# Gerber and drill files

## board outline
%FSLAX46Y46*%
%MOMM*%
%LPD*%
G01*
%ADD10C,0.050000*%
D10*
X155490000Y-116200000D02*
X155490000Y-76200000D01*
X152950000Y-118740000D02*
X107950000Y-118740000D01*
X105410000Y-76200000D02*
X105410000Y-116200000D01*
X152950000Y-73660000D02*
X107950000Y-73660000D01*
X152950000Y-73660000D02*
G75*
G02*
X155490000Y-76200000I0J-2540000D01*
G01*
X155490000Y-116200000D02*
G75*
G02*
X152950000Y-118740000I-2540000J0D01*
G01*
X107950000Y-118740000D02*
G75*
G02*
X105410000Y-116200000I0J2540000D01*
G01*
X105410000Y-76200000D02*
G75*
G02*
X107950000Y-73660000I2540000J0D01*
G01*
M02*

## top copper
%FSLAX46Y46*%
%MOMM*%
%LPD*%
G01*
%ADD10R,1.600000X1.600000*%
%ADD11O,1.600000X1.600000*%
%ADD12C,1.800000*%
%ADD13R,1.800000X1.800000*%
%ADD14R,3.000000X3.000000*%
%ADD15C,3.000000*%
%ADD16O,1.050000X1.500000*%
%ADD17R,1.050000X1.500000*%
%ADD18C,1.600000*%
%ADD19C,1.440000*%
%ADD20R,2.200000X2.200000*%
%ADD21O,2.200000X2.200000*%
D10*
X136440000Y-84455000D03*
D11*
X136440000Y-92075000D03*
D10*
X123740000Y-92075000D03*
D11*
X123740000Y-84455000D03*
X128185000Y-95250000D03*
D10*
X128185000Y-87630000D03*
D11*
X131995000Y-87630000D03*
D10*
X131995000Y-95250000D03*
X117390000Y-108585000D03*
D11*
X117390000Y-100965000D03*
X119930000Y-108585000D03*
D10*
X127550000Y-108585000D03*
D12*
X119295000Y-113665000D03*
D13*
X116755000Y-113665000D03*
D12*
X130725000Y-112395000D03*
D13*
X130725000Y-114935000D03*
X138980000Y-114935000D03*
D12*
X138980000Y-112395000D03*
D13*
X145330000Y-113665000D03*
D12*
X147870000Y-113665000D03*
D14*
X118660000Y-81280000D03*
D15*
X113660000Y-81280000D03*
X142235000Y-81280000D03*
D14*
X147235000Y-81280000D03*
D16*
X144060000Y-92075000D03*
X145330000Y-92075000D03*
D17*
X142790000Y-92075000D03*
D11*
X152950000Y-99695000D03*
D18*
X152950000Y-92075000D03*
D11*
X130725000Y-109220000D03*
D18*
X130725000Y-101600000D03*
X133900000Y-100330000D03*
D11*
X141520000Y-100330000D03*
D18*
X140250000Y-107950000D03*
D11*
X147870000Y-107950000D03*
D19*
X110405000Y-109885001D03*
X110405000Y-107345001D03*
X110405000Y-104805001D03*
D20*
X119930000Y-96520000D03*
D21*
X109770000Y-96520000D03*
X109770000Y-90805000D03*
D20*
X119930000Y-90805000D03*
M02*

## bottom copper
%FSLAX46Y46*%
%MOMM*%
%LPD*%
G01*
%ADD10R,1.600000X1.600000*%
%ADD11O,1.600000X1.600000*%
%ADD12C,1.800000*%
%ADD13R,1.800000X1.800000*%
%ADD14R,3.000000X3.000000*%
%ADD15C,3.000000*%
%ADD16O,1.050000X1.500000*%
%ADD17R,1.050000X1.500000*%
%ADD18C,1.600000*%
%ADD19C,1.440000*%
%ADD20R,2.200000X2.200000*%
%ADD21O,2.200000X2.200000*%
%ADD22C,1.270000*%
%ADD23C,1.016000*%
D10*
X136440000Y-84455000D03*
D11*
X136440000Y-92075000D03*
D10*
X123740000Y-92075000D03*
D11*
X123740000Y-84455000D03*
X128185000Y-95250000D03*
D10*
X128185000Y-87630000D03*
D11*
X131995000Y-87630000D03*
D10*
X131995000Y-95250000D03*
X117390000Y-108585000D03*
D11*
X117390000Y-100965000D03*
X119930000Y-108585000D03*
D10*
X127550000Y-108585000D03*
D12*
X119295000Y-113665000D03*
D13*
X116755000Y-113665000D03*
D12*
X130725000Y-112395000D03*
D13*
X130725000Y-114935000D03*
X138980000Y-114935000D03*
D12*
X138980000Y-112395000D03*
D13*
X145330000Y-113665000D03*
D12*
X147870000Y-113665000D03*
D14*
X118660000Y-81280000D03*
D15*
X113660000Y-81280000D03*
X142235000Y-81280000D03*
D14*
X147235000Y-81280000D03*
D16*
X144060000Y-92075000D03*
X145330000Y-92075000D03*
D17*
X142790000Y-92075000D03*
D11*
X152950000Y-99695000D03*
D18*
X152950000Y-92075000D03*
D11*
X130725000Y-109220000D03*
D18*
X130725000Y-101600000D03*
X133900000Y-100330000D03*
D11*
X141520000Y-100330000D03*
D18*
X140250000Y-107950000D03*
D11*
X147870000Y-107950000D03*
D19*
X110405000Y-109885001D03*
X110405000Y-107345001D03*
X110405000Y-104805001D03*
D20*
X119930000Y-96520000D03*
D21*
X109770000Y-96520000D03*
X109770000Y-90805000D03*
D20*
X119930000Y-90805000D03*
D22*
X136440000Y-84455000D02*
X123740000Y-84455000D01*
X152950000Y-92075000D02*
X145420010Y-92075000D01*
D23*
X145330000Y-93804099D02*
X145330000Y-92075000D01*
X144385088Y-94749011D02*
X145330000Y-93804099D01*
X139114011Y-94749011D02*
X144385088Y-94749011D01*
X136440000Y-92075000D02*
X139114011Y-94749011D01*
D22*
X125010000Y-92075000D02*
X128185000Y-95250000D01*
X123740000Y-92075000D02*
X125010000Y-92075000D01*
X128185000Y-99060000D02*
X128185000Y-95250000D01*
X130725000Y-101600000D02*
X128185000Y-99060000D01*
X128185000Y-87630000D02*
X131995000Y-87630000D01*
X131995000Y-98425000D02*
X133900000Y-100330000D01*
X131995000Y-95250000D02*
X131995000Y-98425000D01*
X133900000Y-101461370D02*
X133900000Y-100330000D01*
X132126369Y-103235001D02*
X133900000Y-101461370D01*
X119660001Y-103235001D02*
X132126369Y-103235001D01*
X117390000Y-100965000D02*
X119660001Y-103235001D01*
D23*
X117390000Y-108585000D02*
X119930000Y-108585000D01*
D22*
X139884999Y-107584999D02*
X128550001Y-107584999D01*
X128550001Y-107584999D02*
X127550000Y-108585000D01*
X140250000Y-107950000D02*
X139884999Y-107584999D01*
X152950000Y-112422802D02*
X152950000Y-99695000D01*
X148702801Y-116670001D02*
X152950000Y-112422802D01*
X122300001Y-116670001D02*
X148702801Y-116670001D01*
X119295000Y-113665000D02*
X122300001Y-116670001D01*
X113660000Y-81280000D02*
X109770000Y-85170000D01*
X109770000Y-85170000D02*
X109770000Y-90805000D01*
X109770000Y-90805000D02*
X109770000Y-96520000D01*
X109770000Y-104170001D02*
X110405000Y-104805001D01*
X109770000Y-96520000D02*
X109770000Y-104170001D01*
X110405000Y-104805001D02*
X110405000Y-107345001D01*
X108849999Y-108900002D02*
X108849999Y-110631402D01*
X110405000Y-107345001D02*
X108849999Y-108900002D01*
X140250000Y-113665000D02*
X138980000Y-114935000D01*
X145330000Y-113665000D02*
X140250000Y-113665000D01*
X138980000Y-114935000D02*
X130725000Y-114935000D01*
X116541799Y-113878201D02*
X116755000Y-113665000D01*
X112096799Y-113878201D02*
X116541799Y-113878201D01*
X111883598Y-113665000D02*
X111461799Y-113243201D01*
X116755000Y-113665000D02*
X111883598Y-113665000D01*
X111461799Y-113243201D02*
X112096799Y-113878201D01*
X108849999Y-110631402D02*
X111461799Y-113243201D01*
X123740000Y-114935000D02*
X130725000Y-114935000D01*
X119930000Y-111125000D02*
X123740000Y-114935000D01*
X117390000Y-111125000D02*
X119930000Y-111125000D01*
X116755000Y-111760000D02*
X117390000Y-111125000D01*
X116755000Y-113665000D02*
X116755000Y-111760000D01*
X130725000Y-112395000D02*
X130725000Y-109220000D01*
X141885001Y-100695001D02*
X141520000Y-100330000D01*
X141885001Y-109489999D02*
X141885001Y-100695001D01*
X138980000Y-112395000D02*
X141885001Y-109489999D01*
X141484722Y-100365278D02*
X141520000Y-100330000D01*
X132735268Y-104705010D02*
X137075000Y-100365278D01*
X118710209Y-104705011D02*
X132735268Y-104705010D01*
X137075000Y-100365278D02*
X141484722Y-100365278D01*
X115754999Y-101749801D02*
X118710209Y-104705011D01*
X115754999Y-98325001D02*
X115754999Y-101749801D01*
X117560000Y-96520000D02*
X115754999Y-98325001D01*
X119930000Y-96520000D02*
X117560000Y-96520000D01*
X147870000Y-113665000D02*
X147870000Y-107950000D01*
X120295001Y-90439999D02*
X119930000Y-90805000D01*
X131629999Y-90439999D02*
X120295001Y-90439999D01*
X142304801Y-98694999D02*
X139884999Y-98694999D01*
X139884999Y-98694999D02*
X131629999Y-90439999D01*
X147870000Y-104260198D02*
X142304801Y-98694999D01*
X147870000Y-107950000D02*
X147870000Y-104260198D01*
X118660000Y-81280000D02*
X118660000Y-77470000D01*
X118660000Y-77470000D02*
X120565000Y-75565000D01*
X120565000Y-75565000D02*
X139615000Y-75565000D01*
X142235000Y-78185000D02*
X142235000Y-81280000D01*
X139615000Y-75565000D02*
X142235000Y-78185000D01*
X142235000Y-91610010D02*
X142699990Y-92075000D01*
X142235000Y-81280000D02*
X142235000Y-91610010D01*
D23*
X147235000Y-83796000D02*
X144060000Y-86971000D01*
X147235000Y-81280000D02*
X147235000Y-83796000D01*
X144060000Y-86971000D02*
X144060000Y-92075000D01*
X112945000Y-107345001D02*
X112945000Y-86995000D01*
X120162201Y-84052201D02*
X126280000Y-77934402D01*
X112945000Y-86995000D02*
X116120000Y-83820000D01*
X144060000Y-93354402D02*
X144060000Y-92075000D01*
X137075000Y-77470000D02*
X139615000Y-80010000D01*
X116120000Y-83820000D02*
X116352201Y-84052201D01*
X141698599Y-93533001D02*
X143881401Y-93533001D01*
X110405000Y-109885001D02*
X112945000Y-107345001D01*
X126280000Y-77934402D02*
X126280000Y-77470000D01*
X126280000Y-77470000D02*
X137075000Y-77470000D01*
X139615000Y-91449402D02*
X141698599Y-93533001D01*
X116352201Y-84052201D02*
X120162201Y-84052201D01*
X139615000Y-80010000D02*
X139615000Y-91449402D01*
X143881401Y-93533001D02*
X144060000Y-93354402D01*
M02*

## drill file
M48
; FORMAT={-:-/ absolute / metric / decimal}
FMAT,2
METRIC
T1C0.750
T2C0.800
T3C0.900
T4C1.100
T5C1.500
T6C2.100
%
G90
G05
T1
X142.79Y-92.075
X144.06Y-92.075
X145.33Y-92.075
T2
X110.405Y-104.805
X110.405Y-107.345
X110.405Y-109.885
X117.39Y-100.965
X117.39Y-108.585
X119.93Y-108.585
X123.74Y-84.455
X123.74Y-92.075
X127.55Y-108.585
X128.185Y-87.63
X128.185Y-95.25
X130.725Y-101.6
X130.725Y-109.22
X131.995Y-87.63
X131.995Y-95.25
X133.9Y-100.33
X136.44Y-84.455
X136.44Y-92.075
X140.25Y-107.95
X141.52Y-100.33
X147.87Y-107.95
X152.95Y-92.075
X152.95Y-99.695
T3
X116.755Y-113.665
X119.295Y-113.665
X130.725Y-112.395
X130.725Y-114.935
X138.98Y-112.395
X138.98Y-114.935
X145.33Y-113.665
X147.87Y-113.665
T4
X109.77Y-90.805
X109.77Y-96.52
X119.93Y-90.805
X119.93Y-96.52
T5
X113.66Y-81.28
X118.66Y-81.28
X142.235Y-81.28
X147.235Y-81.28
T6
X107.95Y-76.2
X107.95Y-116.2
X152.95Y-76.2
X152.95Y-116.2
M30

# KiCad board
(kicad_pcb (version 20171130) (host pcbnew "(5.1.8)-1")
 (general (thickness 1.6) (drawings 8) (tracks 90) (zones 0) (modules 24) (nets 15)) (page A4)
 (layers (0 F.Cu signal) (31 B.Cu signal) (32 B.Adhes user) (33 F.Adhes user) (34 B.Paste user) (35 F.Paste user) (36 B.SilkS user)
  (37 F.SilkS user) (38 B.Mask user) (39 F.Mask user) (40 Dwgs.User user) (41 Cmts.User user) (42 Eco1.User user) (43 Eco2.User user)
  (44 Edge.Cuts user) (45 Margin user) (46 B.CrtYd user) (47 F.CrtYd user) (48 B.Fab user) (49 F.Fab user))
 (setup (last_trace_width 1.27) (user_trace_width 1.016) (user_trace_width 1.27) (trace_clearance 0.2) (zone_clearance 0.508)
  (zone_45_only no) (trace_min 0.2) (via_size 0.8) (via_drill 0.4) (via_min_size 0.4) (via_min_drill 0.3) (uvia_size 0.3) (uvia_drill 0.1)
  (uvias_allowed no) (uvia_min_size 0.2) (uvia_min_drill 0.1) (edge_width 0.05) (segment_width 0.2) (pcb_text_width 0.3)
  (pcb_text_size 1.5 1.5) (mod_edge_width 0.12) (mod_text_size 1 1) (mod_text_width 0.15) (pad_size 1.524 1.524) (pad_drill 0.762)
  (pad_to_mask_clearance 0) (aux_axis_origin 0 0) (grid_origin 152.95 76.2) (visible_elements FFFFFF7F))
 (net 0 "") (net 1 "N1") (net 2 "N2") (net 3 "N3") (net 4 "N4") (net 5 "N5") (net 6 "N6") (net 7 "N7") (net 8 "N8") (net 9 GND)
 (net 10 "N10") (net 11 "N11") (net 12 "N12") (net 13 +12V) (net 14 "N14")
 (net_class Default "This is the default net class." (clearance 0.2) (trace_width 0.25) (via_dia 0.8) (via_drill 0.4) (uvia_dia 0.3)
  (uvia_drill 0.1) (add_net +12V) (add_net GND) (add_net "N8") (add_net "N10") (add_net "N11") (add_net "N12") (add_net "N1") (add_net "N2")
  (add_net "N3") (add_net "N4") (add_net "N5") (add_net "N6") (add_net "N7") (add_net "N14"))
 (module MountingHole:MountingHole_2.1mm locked (layer F.Cu) (at 152.95 116.2)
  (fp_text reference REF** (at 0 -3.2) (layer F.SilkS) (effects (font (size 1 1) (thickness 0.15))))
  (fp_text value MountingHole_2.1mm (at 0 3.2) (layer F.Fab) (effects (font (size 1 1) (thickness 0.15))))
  (pad "" np_thru_hole circle (at 0 0) (size 2.1 2.1) (drill 2.1) (layers *.Cu *.Mask)))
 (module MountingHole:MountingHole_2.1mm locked (layer F.Cu) (at 107.95 116.2)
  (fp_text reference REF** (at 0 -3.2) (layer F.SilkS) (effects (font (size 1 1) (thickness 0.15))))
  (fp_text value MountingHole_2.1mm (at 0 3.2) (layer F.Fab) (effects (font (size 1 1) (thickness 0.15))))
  (pad "" np_thru_hole circle (at 0 0) (size 2.1 2.1) (drill 2.1) (layers *.Cu *.Mask)))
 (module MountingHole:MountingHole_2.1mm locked (layer F.Cu) (at 152.95 76.2)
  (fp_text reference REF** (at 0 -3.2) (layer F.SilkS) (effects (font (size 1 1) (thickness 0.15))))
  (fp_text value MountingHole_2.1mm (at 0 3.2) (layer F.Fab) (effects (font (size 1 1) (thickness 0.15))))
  (pad "" np_thru_hole circle (at 0 0) (size 2.1 2.1) (drill 2.1) (layers *.Cu *.Mask)))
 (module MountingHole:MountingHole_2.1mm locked (layer F.Cu) (at 107.95 76.2)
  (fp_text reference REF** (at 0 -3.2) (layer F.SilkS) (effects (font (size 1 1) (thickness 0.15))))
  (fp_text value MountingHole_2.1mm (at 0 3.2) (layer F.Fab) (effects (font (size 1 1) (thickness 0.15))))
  (pad "" np_thru_hole circle (at 0 0) (size 2.1 2.1) (drill 2.1) (layers *.Cu *.Mask)))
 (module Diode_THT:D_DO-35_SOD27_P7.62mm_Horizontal (layer F.Cu) (at 136.44 84.455 270)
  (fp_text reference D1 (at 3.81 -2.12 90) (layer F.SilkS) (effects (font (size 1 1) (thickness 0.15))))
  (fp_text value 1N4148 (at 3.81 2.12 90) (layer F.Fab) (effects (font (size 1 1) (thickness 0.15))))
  (pad 1 thru_hole rect (at 0 0 270) (size 1.6 1.6) (drill 0.8) (layers *.Cu *.Mask) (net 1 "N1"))
  (pad 2 thru_hole oval (at 7.62 0 270) (size 1.6 1.6) (drill 0.8) (layers *.Cu *.Mask) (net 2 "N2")))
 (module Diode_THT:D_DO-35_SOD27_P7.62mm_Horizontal (layer F.Cu) (at 123.74 92.075 90)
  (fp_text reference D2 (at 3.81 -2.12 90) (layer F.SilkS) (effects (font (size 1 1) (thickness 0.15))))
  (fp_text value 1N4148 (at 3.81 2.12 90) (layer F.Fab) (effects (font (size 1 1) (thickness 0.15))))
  (pad 1 thru_hole rect (at 0 0 90) (size 1.6 1.6) (drill 0.8) (layers *.Cu *.Mask) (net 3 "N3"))
  (pad 2 thru_hole oval (at 7.62 0 90) (size 1.6 1.6) (drill 0.8) (layers *.Cu *.Mask) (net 1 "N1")))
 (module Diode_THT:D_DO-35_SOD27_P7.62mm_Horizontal (layer F.Cu) (at 128.185 87.63 270)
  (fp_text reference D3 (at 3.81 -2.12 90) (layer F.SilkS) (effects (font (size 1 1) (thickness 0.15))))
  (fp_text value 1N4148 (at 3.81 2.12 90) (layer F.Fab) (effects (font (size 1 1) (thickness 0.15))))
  (pad 2 thru_hole oval (at 7.62 0 270) (size 1.6 1.6) (drill 0.8) (layers *.Cu *.Mask) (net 3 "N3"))
  (pad 1 thru_hole rect (at 0 0 270) (size 1.6 1.6) (drill 0.8) (layers *.Cu *.Mask) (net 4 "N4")))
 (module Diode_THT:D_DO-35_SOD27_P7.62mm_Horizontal (layer F.Cu) (at 131.995 95.25 90)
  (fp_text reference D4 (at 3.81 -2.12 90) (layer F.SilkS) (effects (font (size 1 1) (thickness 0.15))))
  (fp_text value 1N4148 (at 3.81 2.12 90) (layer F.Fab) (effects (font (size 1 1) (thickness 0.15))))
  (pad 2 thru_hole oval (at 7.62 0 90) (size 1.6 1.6) (drill 0.8) (layers *.Cu *.Mask) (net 4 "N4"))
  (pad 1 thru_hole rect (at 0 0 90) (size 1.6 1.6) (drill 0.8) (layers *.Cu *.Mask) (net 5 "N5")))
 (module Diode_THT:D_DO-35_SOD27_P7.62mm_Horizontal (layer F.Cu) (at 117.39 108.585 90)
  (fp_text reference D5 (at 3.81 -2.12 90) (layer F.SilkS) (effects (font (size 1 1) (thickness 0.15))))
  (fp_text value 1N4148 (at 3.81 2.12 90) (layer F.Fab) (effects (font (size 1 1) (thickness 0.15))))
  (pad 1 thru_hole rect (at 0 0 90) (size 1.6 1.6) (drill 0.8) (layers *.Cu *.Mask) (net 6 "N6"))
  (pad 2 thru_hole oval (at 7.62 0 90) (size 1.6 1.6) (drill 0.8) (layers *.Cu *.Mask) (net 5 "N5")))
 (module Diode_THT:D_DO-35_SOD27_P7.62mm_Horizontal (layer F.Cu) (at 127.55 108.585 180)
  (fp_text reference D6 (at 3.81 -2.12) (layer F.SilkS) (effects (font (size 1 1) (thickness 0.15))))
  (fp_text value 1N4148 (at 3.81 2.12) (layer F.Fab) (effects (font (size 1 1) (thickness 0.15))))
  (pad 2 thru_hole oval (at 7.62 0 180) (size 1.6 1.6) (drill 0.8) (layers *.Cu *.Mask) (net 6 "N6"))
  (pad 1 thru_hole rect (at 0 0 180) (size 1.6 1.6) (drill 0.8) (layers *.Cu *.Mask) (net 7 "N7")))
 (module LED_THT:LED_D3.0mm (layer F.Cu) (at 116.755 113.665)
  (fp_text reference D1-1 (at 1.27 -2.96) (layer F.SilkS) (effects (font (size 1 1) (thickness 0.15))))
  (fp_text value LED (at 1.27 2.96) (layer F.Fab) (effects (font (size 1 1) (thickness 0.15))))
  (pad 2 thru_hole circle (at 2.54 0) (size 1.8 1.8) (drill 0.9) (layers *.Cu *.Mask) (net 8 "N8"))
  (pad 1 thru_hole rect (at 0 0) (size 1.8 1.8) (drill 0.9) (layers *.Cu *.Mask) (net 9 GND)))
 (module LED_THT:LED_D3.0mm (layer F.Cu) (at 130.725 114.935 90)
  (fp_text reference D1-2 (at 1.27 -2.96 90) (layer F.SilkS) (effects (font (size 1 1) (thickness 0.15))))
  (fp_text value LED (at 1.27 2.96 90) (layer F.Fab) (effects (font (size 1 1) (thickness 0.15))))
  (pad 2 thru_hole circle (at 2.54 0 90) (size 1.8 1.8) (drill 0.9) (layers *.Cu *.Mask) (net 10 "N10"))
  (pad 1 thru_hole rect (at 0 0 90) (size 1.8 1.8) (drill 0.9) (layers *.Cu *.Mask) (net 9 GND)))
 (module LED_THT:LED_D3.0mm (layer F.Cu) (at 138.98 114.935 90)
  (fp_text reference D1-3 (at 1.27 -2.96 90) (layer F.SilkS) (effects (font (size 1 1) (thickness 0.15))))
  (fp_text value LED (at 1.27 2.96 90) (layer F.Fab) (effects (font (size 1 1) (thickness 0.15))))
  (pad 1 thru_hole rect (at 0 0 90) (size 1.8 1.8) (drill 0.9) (layers *.Cu *.Mask) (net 9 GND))
  (pad 2 thru_hole circle (at 2.54 0 90) (size 1.8 1.8) (drill 0.9) (layers *.Cu *.Mask) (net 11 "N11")))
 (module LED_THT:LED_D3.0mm (layer F.Cu) (at 145.33 113.665)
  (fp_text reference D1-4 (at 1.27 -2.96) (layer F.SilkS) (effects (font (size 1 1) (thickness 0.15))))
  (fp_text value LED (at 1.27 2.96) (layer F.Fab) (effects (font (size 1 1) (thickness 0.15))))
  (pad 1 thru_hole rect (at 0 0) (size 1.8 1.8) (drill 0.9) (layers *.Cu *.Mask) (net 9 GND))
  (pad 2 thru_hole circle (at 2.54 0) (size 1.8 1.8) (drill 0.9) (layers *.Cu *.Mask) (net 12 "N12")))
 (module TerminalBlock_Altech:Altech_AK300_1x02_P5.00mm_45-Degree (layer F.Cu) (at 118.66 81.28 180)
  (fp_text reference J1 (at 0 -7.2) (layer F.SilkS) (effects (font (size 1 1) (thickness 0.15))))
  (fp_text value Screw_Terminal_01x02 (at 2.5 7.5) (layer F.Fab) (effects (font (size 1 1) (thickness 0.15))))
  (pad 1 thru_hole rect (at 0 0 180) (size 3 3) (drill 1.5) (layers *.Cu *.Mask) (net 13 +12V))
  (pad 2 thru_hole circle (at 5 0 180) (size 3 3) (drill 1.5) (layers *.Cu *.Mask) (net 9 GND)))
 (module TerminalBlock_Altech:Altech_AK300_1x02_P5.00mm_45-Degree (layer F.Cu) (at 147.235 81.28 180)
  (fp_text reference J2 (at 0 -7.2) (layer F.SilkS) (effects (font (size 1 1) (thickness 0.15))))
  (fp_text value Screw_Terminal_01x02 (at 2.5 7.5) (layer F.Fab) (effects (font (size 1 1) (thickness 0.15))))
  (pad 2 thru_hole circle (at 5 0 180) (size 3 3) (drill 1.5) (layers *.Cu *.Mask) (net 13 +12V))
  (pad 1 thru_hole rect (at 0 0 180) (size 3 3) (drill 1.5) (layers *.Cu *.Mask) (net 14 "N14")))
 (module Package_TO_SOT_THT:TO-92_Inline (layer F.Cu) (at 142.79 92.075)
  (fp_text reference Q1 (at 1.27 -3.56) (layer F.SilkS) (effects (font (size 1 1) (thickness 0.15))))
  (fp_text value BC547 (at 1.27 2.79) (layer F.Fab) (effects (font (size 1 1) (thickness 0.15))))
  (pad 2 thru_hole oval (at 1.27 0) (size 1.05 1.5) (drill 0.75) (layers *.Cu *.Mask) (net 14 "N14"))
  (pad 3 thru_hole oval (at 2.54 0) (size 1.05 1.5) (drill 0.75) (layers *.Cu *.Mask) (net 2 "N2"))
  (pad 1 thru_hole rect (at 0 0) (size 1.05 1.5) (drill 0.75) (layers *.Cu *.Mask) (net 13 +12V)))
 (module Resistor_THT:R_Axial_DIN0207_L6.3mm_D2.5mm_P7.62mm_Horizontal (layer F.Cu) (at 152.95 92.075 270)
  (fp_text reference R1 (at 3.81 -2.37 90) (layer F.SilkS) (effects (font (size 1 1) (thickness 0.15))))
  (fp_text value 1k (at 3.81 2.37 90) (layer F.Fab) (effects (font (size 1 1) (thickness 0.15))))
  (pad 2 thru_hole oval (at 7.62 0 270) (size 1.6 1.6) (drill 0.8) (layers *.Cu *.Mask) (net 8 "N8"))
  (pad 1 thru_hole circle (at 0 0 270) (size 1.6 1.6) (drill 0.8) (layers *.Cu *.Mask) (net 2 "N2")))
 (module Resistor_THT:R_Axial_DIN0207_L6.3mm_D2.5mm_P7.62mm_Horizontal (layer F.Cu) (at 130.725 101.6 270)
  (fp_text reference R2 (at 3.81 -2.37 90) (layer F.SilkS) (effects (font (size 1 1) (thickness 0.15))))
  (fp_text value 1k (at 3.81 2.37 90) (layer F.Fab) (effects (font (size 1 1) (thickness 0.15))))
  (pad 2 thru_hole oval (at 7.62 0 270) (size 1.6 1.6) (drill 0.8) (layers *.Cu *.Mask) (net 10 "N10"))
  (pad 1 thru_hole circle (at 0 0 270) (size 1.6 1.6) (drill 0.8) (layers *.Cu *.Mask) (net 3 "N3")))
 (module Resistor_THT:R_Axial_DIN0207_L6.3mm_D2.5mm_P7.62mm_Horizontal (layer F.Cu) (at 133.9 100.33)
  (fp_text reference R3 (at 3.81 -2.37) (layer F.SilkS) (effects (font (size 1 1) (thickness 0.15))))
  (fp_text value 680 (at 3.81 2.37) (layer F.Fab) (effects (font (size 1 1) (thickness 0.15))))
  (pad 1 thru_hole circle (at 0 0) (size 1.6 1.6) (drill 0.8) (layers *.Cu *.Mask) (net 5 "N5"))
  (pad 2 thru_hole oval (at 7.62 0) (size 1.6 1.6) (drill 0.8) (layers *.Cu *.Mask) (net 11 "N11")))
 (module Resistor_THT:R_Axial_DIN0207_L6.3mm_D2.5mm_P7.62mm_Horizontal (layer F.Cu) (at 140.25 107.95)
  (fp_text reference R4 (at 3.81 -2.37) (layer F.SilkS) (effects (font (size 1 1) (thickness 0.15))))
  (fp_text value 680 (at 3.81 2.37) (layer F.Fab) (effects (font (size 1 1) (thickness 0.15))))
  (pad 1 thru_hole circle (at 0 0) (size 1.6 1.6) (drill 0.8) (layers *.Cu *.Mask) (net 7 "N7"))
  (pad 2 thru_hole oval (at 7.62 0) (size 1.6 1.6) (drill 0.8) (layers *.Cu *.Mask) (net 12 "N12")))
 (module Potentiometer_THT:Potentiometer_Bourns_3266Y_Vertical (layer F.Cu) (at 110.405 109.885001 270)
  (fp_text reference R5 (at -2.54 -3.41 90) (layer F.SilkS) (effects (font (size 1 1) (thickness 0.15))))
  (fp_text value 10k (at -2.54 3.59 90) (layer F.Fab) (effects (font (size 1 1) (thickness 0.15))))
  (pad 1 thru_hole circle (at 0 0 270) (size 1.44 1.44) (drill 0.8) (layers *.Cu *.Mask) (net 14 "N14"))
  (pad 2 thru_hole circle (at -2.54 0 270) (size 1.44 1.44) (drill 0.8) (layers *.Cu *.Mask) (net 9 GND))
  (pad 3 thru_hole circle (at -5.08 0 270) (size 1.44 1.44) (drill 0.8) (layers *.Cu *.Mask) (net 9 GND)))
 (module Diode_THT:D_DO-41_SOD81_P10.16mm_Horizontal (layer F.Cu) (at 119.93 96.52 180)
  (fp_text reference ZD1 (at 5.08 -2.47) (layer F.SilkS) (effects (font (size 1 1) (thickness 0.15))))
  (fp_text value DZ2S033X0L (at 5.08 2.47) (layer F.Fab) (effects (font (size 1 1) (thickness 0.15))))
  (pad 1 thru_hole rect (at 0 0 180) (size 2.2 2.2) (drill 1.1) (layers *.Cu *.Mask) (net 11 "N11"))
  (pad 2 thru_hole oval (at 10.16 0 180) (size 2.2 2.2) (drill 1.1) (layers *.Cu *.Mask) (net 9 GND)))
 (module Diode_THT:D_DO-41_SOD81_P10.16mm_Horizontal (layer F.Cu) (at 119.93 90.805 180)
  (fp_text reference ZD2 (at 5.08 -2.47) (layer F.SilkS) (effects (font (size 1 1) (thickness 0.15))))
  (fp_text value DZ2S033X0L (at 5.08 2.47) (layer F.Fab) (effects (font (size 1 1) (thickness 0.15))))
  (pad 2 thru_hole oval (at 10.16 0 180) (size 2.2 2.2) (drill 1.1) (layers *.Cu *.Mask) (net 9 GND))
  (pad 1 thru_hole rect (at 0 0 180) (size 2.2 2.2) (drill 1.1) (layers *.Cu *.Mask) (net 12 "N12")))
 (gr_line (start 155.49 116.2) (end 155.49 76.2) (layer Edge.Cuts) (width 0.05))
 (gr_line (start 152.95 118.74) (end 107.95 118.74) (layer Edge.Cuts) (width 0.05))
 (gr_line (start 105.41 76.2) (end 105.41 116.2) (layer Edge.Cuts) (width 0.05))
 (gr_line (start 152.95 73.66) (end 107.95 73.66) (layer Edge.Cuts) (width 0.05))
 (gr_arc (start 152.95 76.2) (end 155.49 76.2) (angle -90) (layer Edge.Cuts) (width 0.05))
 (gr_arc (start 152.95 116.2) (end 152.95 118.74) (angle -90) (layer Edge.Cuts) (width 0.05))
 (gr_arc (start 107.95 116.2) (end 105.41 116.2) (angle -90) (layer Edge.Cuts) (width 0.05))
 (gr_arc (start 107.95 76.2) (end 107.95 73.66) (angle -90) (layer Edge.Cuts) (width 0.05))
 (segment (start 136.44 84.455) (end 123.74 84.455) (width 1.27) (layer B.Cu) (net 1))
 (segment (start 152.95 92.075) (end 145.42001 92.075) (width 1.27) (layer B.Cu) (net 2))
 (segment (start 145.33 93.804099) (end 145.33 92.075) (width 1.016) (layer B.Cu) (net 2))
 (segment (start 144.385088 94.749011) (end 145.33 93.804099) (width 1.016) (layer B.Cu) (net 2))
 (segment (start 139.114011 94.749011) (end 144.385088 94.749011) (width 1.016) (layer B.Cu) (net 2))
 (segment (start 136.44 92.075) (end 139.114011 94.749011) (width 1.016) (layer B.Cu) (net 2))
 (segment (start 125.01 92.075) (end 128.185 95.25) (width 1.27) (layer B.Cu) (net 3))
 (segment (start 123.74 92.075) (end 125.01 92.075) (width 1.27) (layer B.Cu) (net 3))
 (segment (start 128.185 99.06) (end 128.185 95.25) (width 1.27) (layer B.Cu) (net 3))
 (segment (start 130.725 101.6) (end 128.185 99.06) (width 1.27) (layer B.Cu) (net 3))
 (segment (start 128.185 87.63) (end 131.995 87.63) (width 1.27) (layer B.Cu) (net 4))
 (segment (start 131.995 98.425) (end 133.9 100.33) (width 1.27) (layer B.Cu) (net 5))
 (segment (start 131.995 95.25) (end 131.995 98.425) (width 1.27) (layer B.Cu) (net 5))
 (segment (start 133.9 101.46137) (end 133.9 100.33) (width 1.27) (layer B.Cu) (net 5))
 (segment (start 132.126369 103.235001) (end 133.9 101.46137) (width 1.27) (layer B.Cu) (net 5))
 (segment (start 119.660001 103.235001) (end 132.126369 103.235001) (width 1.27) (layer B.Cu) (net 5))
 (segment (start 117.39 100.965) (end 119.660001 103.235001) (width 1.27) (layer B.Cu) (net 5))
 (segment (start 117.39 108.585) (end 119.93 108.585) (width 1.016) (layer B.Cu) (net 6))
 (segment (start 139.884999 107.584999) (end 128.550001 107.584999) (width 1.27) (layer B.Cu) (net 7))
 (segment (start 128.550001 107.584999) (end 127.55 108.585) (width 1.27) (layer B.Cu) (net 7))
 (segment (start 140.25 107.95) (end 139.884999 107.584999) (width 1.27) (layer B.Cu) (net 7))
 (segment (start 152.95 112.422802) (end 152.95 99.695) (width 1.27) (layer B.Cu) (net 8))
 (segment (start 148.702801 116.670001) (end 152.95 112.422802) (width 1.27) (layer B.Cu) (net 8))
 (segment (start 122.300001 116.670001) (end 148.702801 116.670001) (width 1.27) (layer B.Cu) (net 8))
 (segment (start 119.295 113.665) (end 122.300001 116.670001) (width 1.27) (layer B.Cu) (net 8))
 (segment (start 113.66 81.28) (end 109.77 85.17) (width 1.27) (layer B.Cu) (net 9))
 (segment (start 109.77 85.17) (end 109.77 90.805) (width 1.27) (layer B.Cu) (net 9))
 (segment (start 109.77 90.805) (end 109.77 96.52) (width 1.27) (layer B.Cu) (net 9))
 (segment (start 109.77 104.170001) (end 110.405 104.805001) (width 1.27) (layer B.Cu) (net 9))
 (segment (start 109.77 96.52) (end 109.77 104.170001) (width 1.27) (layer B.Cu) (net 9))
 (segment (start 110.405 104.805001) (end 110.405 107.345001) (width 1.27) (layer B.Cu) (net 9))
 (segment (start 108.849999 108.900002) (end 108.849999 110.631402) (width 1.27) (layer B.Cu) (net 9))
 (segment (start 110.405 107.345001) (end 108.849999 108.900002) (width 1.27) (layer B.Cu) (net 9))
 (segment (start 140.25 113.665) (end 138.98 114.935) (width 1.27) (layer B.Cu) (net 9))
 (segment (start 145.33 113.665) (end 140.25 113.665) (width 1.27) (layer B.Cu) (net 9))
 (segment (start 138.98 114.935) (end 130.725 114.935) (width 1.27) (layer B.Cu) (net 9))
 (segment (start 116.541799 113.878201) (end 116.755 113.665) (width 1.27) (layer B.Cu) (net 9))
 (segment (start 112.096799 113.878201) (end 116.541799 113.878201) (width 1.27) (layer B.Cu) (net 9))
 (segment (start 111.883598 113.665) (end 111.461799 113.243201) (width 1.27) (layer B.Cu) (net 9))
 (segment (start 116.755 113.665) (end 111.883598 113.665) (width 1.27) (layer B.Cu) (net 9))
 (segment (start 111.461799 113.243201) (end 112.096799 113.878201) (width 1.27) (layer B.Cu) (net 9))
 (segment (start 108.849999 110.631402) (end 111.461799 113.243201) (width 1.27) (layer B.Cu) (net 9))
 (segment (start 123.74 114.935) (end 130.725 114.935) (width 1.27) (layer B.Cu) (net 9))
 (segment (start 119.93 111.125) (end 123.74 114.935) (width 1.27) (layer B.Cu) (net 9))
 (segment (start 117.39 111.125) (end 119.93 111.125) (width 1.27) (layer B.Cu) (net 9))
 (segment (start 116.755 111.76) (end 117.39 111.125) (width 1.27) (layer B.Cu) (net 9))
 (segment (start 116.755 113.665) (end 116.755 111.76) (width 1.27) (layer B.Cu) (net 9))
 (segment (start 130.725 112.395) (end 130.725 109.22) (width 1.27) (layer B.Cu) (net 10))
 (segment (start 141.885001 100.695001) (end 141.52 100.33) (width 1.27) (layer B.Cu) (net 11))
 (segment (start 141.885001 109.489999) (end 141.885001 100.695001) (width 1.27) (layer B.Cu) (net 11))
 (segment (start 138.98 112.395) (end 141.885001 109.489999) (width 1.27) (layer B.Cu) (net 11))
 (segment (start 141.484722 100.365278) (end 141.52 100.33) (width 1.27) (layer B.Cu) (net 11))
 (segment (start 132.735268 104.70501) (end 137.075 100.365278) (width 1.27) (layer B.Cu) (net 11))
 (segment (start 118.710209 104.705011) (end 132.735268 104.70501) (width 1.27) (layer B.Cu) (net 11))
 (segment (start 137.075 100.365278) (end 141.484722 100.365278) (width 1.27) (layer B.Cu) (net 11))
 (segment (start 115.754999 101.749801) (end 118.710209 104.705011) (width 1.27) (layer B.Cu) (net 11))
 (segment (start 115.754999 98.325001) (end 115.754999 101.749801) (width 1.27) (layer B.Cu) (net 11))
 (segment (start 117.56 96.52) (end 115.754999 98.325001) (width 1.27) (layer B.Cu) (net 11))
 (segment (start 119.93 96.52) (end 117.56 96.52) (width 1.27) (layer B.Cu) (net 11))
 (segment (start 147.87 113.665) (end 147.87 107.95) (width 1.27) (layer B.Cu) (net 12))
 (segment (start 120.295001 90.439999) (end 119.93 90.805) (width 1.27) (layer B.Cu) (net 12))
 (segment (start 131.629999 90.439999) (end 120.295001 90.439999) (width 1.27) (layer B.Cu) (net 12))
 (segment (start 142.304801 98.694999) (end 139.884999 98.694999) (width 1.27) (layer B.Cu) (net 12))
 (segment (start 139.884999 98.694999) (end 131.629999 90.439999) (width 1.27) (layer B.Cu) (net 12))
 (segment (start 147.87 104.260198) (end 142.304801 98.694999) (width 1.27) (layer B.Cu) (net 12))
 (segment (start 147.87 107.95) (end 147.87 104.260198) (width 1.27) (layer B.Cu) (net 12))
 (segment (start 118.66 81.28) (end 118.66 77.47) (width 1.27) (layer B.Cu) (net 13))
 (segment (start 118.66 77.47) (end 120.565 75.565) (width 1.27) (layer B.Cu) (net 13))
 (segment (start 120.565 75.565) (end 139.615 75.565) (width 1.27) (layer B.Cu) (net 13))
 (segment (start 142.235 78.185) (end 142.235 81.28) (width 1.27) (layer B.Cu) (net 13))
 (segment (start 139.615 75.565) (end 142.235 78.185) (width 1.27) (layer B.Cu) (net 13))
 (segment (start 142.235 91.61001) (end 142.69999 92.075) (width 1.27) (layer B.Cu) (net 13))
 (segment (start 142.235 81.28) (end 142.235 91.61001) (width 1.27) (layer B.Cu) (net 13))
 (segment (start 147.235 83.796) (end 144.06 86.971) (width 1.016) (layer B.Cu) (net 14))
 (segment (start 147.235 81.28) (end 147.235 83.796) (width 1.016) (layer B.Cu) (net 14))
 (segment (start 144.06 86.971) (end 144.06 92.075) (width 1.016) (layer B.Cu) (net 14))
 (segment (start 112.945 107.345001) (end 112.945 86.995) (width 1.016) (layer B.Cu) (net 14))
 (segment (start 120.162201 84.052201) (end 126.28 77.934402) (width 1.016) (layer B.Cu) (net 14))
 (segment (start 112.945 86.995) (end 116.12 83.82) (width 1.016) (layer B.Cu) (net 14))
 (segment (start 144.06 93.354402) (end 144.06 92.075) (width 1.016) (layer B.Cu) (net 14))
 (segment (start 137.075 77.47) (end 139.615 80.01) (width 1.016) (layer B.Cu) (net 14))
 (segment (start 116.12 83.82) (end 116.352201 84.052201) (width 1.016) (layer B.Cu) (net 14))
 (segment (start 141.698599 93.533001) (end 143.881401 93.533001) (width 1.016) (layer B.Cu) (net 14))
 (segment (start 110.405 109.885001) (end 112.945 107.345001) (width 1.016) (layer B.Cu) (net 14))
 (segment (start 126.28 77.934402) (end 126.28 77.47) (width 1.016) (layer B.Cu) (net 14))
 (segment (start 126.28 77.47) (end 137.075 77.47) (width 1.016) (layer B.Cu) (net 14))
 (segment (start 139.615 91.449402) (end 141.698599 93.533001) (width 1.016) (layer B.Cu) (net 14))
 (segment (start 116.352201 84.052201) (end 120.162201 84.052201) (width 1.016) (layer B.Cu) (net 14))
 (segment (start 139.615 80.01) (end 139.615 91.449402) (width 1.016) (layer B.Cu) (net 14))
 (segment (start 143.881401 93.533001) (end 144.06 93.354402) (width 1.016) (layer B.Cu) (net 14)))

